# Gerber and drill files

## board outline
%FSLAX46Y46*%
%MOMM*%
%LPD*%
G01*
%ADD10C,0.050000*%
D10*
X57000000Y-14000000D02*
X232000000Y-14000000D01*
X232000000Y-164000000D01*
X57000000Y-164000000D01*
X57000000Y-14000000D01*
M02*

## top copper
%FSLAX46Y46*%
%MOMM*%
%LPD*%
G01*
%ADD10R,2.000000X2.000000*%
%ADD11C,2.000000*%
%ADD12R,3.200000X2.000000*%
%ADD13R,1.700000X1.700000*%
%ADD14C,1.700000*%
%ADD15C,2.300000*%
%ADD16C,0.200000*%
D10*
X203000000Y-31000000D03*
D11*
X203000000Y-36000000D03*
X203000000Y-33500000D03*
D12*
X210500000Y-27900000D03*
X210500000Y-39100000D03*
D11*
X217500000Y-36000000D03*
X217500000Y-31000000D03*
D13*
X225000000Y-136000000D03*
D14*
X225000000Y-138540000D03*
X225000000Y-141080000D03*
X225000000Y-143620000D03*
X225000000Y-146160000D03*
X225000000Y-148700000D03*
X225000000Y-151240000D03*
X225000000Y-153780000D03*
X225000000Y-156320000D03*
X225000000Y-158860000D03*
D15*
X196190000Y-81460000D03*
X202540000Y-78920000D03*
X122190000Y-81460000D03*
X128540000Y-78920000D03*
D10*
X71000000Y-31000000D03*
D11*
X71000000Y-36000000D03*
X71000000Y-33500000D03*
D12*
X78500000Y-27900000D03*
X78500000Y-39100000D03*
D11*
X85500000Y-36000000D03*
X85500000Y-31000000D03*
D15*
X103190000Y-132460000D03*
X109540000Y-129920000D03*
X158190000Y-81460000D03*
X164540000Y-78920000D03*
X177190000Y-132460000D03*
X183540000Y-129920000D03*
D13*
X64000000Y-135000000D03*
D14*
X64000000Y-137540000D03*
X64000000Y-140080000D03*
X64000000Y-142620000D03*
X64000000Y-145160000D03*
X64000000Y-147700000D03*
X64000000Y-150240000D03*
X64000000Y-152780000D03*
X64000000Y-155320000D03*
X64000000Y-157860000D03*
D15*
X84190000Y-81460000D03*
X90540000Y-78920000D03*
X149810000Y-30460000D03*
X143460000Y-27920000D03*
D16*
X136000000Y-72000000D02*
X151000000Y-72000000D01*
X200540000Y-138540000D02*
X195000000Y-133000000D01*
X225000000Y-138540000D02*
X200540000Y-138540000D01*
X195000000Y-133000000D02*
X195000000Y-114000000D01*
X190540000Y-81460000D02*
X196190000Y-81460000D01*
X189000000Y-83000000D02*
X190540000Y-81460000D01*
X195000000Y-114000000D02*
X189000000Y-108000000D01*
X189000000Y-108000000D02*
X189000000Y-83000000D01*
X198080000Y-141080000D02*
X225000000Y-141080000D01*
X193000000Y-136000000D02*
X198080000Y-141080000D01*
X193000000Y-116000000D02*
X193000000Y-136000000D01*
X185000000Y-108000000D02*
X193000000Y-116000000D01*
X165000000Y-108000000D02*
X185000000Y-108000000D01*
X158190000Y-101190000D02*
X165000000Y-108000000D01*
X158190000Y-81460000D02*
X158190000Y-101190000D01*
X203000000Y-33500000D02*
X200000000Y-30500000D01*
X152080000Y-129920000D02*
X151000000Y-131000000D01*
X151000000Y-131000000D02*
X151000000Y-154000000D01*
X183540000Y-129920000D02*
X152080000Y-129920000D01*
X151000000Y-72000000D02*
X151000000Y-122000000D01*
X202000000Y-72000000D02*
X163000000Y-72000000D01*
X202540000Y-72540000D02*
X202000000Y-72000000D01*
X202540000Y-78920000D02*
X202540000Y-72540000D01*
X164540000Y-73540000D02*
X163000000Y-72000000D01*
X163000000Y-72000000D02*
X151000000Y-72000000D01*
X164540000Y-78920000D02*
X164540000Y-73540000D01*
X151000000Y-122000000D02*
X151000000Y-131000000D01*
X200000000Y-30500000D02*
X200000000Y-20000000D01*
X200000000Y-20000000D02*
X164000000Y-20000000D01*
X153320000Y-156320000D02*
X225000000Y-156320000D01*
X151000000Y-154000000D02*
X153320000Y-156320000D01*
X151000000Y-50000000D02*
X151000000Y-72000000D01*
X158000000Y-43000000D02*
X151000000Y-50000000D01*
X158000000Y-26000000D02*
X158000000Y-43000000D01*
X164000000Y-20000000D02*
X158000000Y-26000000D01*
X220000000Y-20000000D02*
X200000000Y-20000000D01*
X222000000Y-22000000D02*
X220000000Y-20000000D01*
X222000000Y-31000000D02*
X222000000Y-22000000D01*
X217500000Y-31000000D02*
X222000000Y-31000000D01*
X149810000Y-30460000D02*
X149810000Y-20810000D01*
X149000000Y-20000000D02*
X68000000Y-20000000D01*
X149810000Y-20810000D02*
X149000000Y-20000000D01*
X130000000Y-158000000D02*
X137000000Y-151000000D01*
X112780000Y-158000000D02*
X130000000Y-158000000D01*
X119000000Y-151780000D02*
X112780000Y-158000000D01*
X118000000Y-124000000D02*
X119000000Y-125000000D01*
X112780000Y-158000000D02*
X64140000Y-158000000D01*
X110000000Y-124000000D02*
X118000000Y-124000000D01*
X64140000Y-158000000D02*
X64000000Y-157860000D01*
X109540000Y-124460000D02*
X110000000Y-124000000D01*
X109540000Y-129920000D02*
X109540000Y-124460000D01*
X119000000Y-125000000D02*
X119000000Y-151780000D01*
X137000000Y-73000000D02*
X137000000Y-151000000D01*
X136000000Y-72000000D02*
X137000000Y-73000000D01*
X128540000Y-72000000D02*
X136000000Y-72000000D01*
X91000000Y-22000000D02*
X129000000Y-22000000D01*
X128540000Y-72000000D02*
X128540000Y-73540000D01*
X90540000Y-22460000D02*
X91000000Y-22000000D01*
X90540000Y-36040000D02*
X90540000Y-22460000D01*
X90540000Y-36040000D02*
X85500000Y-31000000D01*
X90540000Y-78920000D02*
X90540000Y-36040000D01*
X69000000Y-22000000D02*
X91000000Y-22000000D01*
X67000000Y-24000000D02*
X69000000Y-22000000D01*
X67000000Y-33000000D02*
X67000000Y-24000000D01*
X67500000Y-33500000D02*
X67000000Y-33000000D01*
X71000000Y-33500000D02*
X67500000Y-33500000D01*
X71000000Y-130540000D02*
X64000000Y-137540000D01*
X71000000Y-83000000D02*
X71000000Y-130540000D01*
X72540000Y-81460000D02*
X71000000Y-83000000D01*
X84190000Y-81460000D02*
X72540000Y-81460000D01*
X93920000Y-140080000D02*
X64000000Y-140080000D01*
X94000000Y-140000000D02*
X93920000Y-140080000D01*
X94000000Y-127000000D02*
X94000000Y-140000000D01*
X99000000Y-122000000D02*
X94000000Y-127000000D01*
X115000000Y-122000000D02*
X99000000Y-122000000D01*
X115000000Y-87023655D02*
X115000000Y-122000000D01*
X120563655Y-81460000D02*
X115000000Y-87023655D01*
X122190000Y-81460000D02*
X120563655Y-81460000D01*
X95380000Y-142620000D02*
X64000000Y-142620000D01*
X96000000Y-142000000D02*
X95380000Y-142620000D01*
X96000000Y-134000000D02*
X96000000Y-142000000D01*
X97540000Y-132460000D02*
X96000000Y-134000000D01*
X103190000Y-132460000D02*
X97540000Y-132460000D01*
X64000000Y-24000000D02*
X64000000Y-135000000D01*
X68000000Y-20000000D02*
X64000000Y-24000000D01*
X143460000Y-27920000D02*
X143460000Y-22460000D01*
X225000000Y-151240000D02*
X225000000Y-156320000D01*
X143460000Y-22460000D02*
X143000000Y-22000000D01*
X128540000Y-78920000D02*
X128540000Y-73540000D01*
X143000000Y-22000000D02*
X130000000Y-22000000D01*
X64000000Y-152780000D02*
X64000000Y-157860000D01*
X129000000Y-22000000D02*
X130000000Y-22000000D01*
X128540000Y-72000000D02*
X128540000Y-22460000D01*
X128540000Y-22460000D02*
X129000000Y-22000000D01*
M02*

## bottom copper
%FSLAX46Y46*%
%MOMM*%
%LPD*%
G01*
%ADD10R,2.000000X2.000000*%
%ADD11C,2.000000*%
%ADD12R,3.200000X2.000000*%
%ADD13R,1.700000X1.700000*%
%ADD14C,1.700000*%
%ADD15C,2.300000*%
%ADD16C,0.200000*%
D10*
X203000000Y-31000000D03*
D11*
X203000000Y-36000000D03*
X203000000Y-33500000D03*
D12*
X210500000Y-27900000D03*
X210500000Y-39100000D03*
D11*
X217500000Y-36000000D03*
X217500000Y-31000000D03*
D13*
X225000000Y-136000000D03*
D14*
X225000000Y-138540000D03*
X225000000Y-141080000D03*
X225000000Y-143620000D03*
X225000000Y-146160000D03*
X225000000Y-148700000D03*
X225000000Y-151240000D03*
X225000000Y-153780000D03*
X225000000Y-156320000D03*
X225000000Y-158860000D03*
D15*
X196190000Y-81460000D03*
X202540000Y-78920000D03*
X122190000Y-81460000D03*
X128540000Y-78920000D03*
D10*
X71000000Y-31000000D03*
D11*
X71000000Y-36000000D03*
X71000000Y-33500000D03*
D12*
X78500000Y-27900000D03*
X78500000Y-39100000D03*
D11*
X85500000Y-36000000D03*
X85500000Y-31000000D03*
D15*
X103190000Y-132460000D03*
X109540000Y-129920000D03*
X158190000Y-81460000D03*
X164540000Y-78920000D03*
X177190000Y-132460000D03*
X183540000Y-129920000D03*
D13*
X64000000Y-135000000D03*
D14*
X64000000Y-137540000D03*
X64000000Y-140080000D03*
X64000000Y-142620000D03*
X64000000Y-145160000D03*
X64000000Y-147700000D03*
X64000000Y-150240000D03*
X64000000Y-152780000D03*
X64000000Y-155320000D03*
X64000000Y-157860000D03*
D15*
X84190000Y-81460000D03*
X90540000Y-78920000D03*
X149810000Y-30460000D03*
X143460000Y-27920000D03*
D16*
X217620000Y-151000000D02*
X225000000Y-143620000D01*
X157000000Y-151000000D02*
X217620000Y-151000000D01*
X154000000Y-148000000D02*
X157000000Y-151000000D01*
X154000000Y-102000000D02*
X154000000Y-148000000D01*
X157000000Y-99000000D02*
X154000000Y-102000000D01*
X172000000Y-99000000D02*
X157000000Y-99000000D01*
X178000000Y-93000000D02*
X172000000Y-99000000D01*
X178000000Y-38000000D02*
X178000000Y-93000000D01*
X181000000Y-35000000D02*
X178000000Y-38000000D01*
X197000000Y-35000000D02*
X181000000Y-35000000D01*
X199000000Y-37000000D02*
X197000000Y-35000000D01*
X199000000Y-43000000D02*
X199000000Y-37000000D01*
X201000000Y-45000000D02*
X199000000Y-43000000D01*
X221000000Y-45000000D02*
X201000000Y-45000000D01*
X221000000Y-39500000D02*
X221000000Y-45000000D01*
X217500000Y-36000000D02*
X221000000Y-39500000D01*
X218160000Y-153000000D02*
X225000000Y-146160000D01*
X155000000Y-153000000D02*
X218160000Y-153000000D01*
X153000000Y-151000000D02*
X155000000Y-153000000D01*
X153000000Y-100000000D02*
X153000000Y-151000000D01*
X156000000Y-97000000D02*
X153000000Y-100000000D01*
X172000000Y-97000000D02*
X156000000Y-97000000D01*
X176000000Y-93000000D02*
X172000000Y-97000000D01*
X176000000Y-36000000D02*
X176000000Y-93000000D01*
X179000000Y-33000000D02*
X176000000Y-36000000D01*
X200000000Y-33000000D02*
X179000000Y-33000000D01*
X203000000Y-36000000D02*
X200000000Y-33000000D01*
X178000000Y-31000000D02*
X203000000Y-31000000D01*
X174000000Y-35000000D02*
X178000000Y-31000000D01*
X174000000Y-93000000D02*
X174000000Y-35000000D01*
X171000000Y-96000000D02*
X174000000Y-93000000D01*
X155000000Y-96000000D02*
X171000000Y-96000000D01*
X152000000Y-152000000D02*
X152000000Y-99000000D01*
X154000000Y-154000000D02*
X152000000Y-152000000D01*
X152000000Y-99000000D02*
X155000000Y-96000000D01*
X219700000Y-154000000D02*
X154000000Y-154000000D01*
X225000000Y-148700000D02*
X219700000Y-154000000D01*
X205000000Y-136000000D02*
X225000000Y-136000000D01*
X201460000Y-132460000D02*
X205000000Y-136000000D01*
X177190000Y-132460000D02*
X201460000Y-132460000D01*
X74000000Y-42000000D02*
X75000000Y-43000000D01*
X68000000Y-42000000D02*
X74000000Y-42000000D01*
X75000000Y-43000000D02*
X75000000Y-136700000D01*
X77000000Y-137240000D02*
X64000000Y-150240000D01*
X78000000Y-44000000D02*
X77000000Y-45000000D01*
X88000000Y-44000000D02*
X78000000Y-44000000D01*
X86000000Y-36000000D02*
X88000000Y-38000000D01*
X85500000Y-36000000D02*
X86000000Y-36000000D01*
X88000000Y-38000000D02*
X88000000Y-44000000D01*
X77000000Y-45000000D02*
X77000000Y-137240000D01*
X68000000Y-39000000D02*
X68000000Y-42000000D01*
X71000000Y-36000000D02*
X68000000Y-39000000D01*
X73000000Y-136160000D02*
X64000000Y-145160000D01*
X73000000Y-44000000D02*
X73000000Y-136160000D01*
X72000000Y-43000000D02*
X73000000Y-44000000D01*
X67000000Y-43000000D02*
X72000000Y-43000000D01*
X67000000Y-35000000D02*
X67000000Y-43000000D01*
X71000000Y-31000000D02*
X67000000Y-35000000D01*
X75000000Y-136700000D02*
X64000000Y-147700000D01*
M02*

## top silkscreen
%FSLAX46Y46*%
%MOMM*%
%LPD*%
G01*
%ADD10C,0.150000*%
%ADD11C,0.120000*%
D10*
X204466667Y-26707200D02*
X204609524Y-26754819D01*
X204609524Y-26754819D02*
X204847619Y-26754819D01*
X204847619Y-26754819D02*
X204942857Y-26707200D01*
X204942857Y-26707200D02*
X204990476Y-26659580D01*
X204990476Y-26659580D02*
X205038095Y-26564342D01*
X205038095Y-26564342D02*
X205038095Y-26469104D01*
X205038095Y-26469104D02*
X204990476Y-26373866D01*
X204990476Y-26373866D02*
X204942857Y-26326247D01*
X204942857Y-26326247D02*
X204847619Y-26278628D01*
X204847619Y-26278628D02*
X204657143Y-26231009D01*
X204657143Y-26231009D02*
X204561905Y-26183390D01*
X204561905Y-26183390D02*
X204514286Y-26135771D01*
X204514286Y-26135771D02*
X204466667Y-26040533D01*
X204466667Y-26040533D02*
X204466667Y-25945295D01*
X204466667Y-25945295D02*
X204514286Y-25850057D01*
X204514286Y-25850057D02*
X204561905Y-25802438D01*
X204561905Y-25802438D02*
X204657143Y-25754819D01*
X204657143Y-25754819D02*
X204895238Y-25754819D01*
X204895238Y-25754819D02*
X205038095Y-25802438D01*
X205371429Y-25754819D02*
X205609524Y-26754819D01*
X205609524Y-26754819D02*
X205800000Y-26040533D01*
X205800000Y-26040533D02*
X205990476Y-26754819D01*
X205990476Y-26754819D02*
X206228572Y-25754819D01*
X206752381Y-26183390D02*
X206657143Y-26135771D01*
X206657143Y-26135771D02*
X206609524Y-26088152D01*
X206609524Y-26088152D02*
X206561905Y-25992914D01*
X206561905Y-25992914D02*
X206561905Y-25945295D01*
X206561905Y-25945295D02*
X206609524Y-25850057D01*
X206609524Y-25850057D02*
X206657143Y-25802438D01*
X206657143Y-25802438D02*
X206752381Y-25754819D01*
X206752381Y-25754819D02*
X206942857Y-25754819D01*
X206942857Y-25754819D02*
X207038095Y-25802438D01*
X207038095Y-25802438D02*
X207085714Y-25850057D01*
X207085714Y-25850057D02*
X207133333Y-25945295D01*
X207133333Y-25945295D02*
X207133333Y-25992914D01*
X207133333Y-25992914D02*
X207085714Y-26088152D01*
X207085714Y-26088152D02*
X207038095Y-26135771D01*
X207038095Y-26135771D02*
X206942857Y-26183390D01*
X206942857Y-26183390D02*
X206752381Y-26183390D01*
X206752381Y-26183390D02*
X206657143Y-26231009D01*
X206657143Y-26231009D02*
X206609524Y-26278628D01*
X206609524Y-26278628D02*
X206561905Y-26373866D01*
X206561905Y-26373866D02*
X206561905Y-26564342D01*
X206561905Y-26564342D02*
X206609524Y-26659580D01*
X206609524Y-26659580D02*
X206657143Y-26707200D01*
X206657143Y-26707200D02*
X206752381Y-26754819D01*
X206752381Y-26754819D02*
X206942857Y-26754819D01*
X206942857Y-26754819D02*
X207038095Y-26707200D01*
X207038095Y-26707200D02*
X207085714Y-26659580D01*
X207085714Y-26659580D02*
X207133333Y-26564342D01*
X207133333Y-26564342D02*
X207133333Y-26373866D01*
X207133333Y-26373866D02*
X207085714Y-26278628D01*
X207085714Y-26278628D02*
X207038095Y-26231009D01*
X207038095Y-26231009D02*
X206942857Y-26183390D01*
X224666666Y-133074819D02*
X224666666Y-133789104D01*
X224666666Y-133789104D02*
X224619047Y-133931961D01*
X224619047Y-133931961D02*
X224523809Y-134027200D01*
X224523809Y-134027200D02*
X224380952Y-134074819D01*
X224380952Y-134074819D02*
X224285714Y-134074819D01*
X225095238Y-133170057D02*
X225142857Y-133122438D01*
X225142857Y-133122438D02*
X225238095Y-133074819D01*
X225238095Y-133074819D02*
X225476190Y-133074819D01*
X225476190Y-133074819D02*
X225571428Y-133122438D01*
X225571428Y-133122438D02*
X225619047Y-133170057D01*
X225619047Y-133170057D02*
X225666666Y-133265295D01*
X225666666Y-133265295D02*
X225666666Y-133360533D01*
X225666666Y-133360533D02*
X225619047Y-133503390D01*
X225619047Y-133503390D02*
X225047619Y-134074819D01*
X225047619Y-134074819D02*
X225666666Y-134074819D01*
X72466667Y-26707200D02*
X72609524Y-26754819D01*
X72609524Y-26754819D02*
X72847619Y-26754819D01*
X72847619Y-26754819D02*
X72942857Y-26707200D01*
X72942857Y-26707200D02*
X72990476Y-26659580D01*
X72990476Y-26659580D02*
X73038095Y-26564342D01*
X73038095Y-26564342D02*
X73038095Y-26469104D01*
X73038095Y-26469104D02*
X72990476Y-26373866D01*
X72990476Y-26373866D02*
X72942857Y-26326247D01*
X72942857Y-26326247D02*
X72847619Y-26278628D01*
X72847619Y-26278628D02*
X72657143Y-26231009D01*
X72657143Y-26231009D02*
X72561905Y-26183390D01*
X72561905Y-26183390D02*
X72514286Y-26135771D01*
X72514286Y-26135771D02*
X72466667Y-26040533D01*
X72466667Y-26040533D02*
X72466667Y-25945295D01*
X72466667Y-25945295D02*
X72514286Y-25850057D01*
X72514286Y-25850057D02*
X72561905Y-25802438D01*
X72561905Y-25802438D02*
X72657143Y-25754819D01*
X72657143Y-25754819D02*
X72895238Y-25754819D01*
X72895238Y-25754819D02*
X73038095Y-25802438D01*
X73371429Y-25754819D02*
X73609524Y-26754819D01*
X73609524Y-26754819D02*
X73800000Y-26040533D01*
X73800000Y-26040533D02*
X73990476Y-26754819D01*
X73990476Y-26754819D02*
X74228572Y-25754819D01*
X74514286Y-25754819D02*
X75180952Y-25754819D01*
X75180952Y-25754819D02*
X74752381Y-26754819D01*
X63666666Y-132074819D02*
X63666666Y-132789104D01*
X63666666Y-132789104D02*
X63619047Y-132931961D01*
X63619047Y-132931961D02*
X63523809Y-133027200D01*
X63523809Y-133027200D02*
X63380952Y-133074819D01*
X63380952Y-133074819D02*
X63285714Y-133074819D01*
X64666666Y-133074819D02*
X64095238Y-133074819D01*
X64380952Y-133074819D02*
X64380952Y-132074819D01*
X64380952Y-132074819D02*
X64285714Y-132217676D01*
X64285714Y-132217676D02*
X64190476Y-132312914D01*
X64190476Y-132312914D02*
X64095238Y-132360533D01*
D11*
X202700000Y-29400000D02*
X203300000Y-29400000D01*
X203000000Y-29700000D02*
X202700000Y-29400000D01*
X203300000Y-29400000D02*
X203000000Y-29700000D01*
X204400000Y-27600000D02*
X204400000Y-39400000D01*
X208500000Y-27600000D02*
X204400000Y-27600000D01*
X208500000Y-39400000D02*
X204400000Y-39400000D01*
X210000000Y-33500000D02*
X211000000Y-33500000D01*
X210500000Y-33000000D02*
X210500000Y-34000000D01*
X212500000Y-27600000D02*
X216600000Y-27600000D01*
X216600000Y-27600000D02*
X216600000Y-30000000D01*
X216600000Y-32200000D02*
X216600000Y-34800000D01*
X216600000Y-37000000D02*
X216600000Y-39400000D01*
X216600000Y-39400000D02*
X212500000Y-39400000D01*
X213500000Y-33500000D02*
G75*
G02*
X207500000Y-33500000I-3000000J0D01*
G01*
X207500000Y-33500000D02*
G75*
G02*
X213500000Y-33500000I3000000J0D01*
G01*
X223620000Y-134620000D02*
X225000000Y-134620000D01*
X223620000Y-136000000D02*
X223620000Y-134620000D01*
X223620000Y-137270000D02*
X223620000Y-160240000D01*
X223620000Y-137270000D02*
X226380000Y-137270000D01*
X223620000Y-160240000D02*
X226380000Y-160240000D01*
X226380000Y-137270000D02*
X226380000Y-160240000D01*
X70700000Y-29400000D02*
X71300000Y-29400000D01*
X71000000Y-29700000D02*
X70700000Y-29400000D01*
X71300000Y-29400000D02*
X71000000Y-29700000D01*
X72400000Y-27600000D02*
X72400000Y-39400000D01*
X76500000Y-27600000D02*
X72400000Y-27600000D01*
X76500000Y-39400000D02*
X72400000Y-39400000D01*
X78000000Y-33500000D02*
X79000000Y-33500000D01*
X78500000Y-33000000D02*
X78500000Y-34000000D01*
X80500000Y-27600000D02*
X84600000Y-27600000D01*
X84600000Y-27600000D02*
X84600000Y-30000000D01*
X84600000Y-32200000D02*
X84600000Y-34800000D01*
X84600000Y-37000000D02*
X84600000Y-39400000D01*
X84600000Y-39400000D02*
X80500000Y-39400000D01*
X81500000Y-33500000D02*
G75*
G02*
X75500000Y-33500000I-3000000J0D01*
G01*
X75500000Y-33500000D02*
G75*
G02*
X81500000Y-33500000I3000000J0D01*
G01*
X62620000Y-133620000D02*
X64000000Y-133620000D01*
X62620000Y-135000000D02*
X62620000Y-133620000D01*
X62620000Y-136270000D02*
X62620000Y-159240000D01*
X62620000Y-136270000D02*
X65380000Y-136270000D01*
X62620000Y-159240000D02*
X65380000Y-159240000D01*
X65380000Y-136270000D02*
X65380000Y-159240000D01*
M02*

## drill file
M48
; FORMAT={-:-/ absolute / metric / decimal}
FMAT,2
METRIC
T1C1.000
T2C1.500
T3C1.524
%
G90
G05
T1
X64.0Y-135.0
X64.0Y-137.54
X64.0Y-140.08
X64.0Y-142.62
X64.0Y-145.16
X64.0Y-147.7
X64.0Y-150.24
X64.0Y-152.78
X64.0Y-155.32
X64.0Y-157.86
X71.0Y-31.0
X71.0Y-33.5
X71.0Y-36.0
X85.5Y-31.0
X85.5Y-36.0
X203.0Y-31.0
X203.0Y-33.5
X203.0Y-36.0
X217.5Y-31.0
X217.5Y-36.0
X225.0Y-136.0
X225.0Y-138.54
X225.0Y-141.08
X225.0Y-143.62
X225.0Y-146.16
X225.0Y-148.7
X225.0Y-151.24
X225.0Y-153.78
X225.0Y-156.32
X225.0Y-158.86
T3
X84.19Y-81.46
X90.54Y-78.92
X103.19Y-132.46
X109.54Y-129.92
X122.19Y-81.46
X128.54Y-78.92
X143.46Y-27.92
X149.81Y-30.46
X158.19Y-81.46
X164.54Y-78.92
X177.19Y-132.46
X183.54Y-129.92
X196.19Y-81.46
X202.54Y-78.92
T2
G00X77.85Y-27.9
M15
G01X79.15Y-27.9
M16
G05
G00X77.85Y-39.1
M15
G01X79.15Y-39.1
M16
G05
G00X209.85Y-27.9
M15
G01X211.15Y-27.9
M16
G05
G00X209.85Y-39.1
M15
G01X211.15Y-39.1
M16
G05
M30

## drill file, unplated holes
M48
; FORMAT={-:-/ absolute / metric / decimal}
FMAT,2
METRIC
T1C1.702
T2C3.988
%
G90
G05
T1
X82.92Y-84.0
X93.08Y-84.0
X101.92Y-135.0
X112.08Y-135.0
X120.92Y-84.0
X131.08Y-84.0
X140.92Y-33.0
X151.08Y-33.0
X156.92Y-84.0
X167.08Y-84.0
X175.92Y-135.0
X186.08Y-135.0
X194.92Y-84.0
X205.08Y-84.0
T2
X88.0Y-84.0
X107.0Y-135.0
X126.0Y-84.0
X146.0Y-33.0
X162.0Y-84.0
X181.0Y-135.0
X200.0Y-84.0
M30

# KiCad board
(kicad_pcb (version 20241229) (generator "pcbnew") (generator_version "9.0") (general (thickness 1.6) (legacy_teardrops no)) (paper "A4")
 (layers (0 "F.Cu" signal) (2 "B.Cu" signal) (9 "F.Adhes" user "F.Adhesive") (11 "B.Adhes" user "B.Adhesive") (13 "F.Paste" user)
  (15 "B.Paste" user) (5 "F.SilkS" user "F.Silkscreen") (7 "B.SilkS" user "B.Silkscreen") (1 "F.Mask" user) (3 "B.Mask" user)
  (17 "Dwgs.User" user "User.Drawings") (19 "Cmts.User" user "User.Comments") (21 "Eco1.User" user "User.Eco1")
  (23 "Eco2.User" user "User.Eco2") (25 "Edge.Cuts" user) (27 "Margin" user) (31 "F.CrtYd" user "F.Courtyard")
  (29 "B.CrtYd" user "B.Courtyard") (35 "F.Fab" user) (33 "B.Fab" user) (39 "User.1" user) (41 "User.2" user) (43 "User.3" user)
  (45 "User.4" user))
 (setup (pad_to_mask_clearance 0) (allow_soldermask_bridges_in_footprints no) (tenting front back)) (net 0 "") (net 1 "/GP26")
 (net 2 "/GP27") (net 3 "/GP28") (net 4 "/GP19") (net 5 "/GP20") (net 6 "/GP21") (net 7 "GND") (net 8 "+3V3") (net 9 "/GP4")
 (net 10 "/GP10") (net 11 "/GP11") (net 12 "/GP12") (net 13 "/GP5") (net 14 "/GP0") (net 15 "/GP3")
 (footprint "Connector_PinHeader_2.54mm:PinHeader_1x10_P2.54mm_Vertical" (layer "F.Cu") (at 225 136)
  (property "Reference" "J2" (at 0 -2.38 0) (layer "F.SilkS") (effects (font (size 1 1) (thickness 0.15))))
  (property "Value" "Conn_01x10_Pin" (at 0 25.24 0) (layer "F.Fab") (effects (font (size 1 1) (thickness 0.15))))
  (fp_line (start -1.38 -1.38) (end 0 -1.38) (stroke (width 0.12) (type solid)) (layer "F.SilkS"))
  (fp_line (start -1.38 0) (end -1.38 -1.38) (stroke (width 0.12) (type solid)) (layer "F.SilkS"))
  (fp_line (start -1.38 1.27) (end -1.38 24.24) (stroke (width 0.12) (type solid)) (layer "F.SilkS"))
  (fp_line (start -1.38 1.27) (end 1.38 1.27) (stroke (width 0.12) (type solid)) (layer "F.SilkS"))
  (fp_line (start -1.38 24.24) (end 1.38 24.24) (stroke (width 0.12) (type solid)) (layer "F.SilkS"))
  (fp_line (start 1.38 1.27) (end 1.38 24.24) (stroke (width 0.12) (type solid)) (layer "F.SilkS"))
  (pad "1" thru_hole rect (at 0 0) (size 1.7 1.7) (drill 1) (layers "*.Cu" "*.Mask") (remove_unused_layers no) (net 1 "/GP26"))
  (pad "2" thru_hole circle (at 0 2.54) (size 1.7 1.7) (drill 1) (layers "*.Cu" "*.Mask") (remove_unused_layers no) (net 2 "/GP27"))
  (pad "3" thru_hole circle (at 0 5.08) (size 1.7 1.7) (drill 1) (layers "*.Cu" "*.Mask") (remove_unused_layers no) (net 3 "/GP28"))
  (pad "4" thru_hole circle (at 0 7.62) (size 1.7 1.7) (drill 1) (layers "*.Cu" "*.Mask") (remove_unused_layers no) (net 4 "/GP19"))
  (pad "5" thru_hole circle (at 0 10.16) (size 1.7 1.7) (drill 1) (layers "*.Cu" "*.Mask") (remove_unused_layers no) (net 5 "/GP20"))
  (pad "6" thru_hole circle (at 0 12.7) (size 1.7 1.7) (drill 1) (layers "*.Cu" "*.Mask") (remove_unused_layers no) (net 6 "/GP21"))
  (pad "7" thru_hole circle (at 0 15.24) (size 1.7 1.7) (drill 1) (layers "*.Cu" "*.Mask") (remove_unused_layers no) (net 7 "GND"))
  (pad "8" thru_hole circle (at 0 17.78) (size 1.7 1.7) (drill 1) (layers "*.Cu" "*.Mask") (remove_unused_layers no) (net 7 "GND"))
  (pad "9" thru_hole circle (at 0 20.32) (size 1.7 1.7) (drill 1) (layers "*.Cu" "*.Mask") (remove_unused_layers no) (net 7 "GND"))
  (pad "10" thru_hole circle (at 0 22.86) (size 1.7 1.7) (drill 1) (layers "*.Cu" "*.Mask") (remove_unused_layers no) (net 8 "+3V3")))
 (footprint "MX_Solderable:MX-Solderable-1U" (layer "F.Cu") (at 200 84)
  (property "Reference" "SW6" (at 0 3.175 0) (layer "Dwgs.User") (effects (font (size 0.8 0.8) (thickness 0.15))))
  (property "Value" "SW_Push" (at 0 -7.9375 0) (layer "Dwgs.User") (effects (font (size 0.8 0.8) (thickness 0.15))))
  (pad "" np_thru_hole circle (at -5.08 0 48.099) (size 1.7018 1.7018) (drill 1.7018) (layers "*.Cu" "*.Mask"))
  (pad "" np_thru_hole circle (at 0 0) (size 3.9878 3.9878) (drill 3.9878) (layers "*.Cu" "*.Mask"))
  (pad "" np_thru_hole circle (at 5.08 0 48.099) (size 1.7018 1.7018) (drill 1.7018) (layers "*.Cu" "*.Mask"))
  (pad "1" thru_hole circle (at -3.81 -2.54) (size 2.3 2.3) (drill 1.524) (layers "*.Cu" "B.Mask") (remove_unused_layers no) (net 2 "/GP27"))
  (pad "2" thru_hole circle (at 2.54 -5.08) (size 2.3 2.3) (drill 1.524) (layers "*.Cu" "B.Mask") (remove_unused_layers no) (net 7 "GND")))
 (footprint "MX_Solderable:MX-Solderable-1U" (layer "F.Cu") (at 126 84)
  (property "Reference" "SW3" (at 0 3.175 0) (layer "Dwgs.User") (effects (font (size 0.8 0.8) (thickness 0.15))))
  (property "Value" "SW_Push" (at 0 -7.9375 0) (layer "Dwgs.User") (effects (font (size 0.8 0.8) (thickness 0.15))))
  (pad "" np_thru_hole circle (at -5.08 0 48.099) (size 1.7018 1.7018) (drill 1.7018) (layers "*.Cu" "*.Mask"))
  (pad "" np_thru_hole circle (at 0 0) (size 3.9878 3.9878) (drill 3.9878) (layers "*.Cu" "*.Mask"))
  (pad "" np_thru_hole circle (at 5.08 0 48.099) (size 1.7018 1.7018) (drill 1.7018) (layers "*.Cu" "*.Mask"))
  (pad "1" thru_hole circle (at -3.81 -2.54) (size 2.3 2.3) (drill 1.524) (layers "*.Cu" "B.Mask") (remove_unused_layers no) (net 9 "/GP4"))
  (pad "2" thru_hole circle (at 2.54 -5.08) (size 2.3 2.3) (drill 1.524) (layers "*.Cu" "B.Mask") (remove_unused_layers no) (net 7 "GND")))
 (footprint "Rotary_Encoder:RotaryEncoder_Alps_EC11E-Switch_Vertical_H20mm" (layer "F.Cu") (at 71 31)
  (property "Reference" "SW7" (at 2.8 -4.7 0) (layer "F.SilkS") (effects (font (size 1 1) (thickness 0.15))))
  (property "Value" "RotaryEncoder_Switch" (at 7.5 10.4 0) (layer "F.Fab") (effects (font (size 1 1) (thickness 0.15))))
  (fp_line (start -0.3 -1.6) (end 0.3 -1.6) (stroke (width 0.12) (type solid)) (layer "F.SilkS"))
  (fp_line (start 0 -1.3) (end -0.3 -1.6) (stroke (width 0.12) (type solid)) (layer "F.SilkS"))
  (fp_line (start 0.3 -1.6) (end 0 -1.3) (stroke (width 0.12) (type solid)) (layer "F.SilkS"))
  (fp_line (start 1.4 -3.4) (end 1.4 8.4) (stroke (width 0.12) (type solid)) (layer "F.SilkS"))
  (fp_line (start 5.5 -3.4) (end 1.4 -3.4) (stroke (width 0.12) (type solid)) (layer "F.SilkS"))
  (fp_line (start 5.5 8.4) (end 1.4 8.4) (stroke (width 0.12) (type solid)) (layer "F.SilkS"))
  (fp_line (start 7 2.5) (end 8 2.5) (stroke (width 0.12) (type solid)) (layer "F.SilkS"))
  (fp_line (start 7.5 2) (end 7.5 3) (stroke (width 0.12) (type solid)) (layer "F.SilkS"))
  (fp_line (start 9.5 -3.4) (end 13.6 -3.4) (stroke (width 0.12) (type solid)) (layer "F.SilkS"))
  (fp_line (start 13.6 -3.4) (end 13.6 -1) (stroke (width 0.12) (type solid)) (layer "F.SilkS"))
  (fp_line (start 13.6 1.2) (end 13.6 3.8) (stroke (width 0.12) (type solid)) (layer "F.SilkS"))
  (fp_line (start 13.6 6) (end 13.6 8.4) (stroke (width 0.12) (type solid)) (layer "F.SilkS"))
  (fp_line (start 13.6 8.4) (end 9.5 8.4) (stroke (width 0.12) (type solid)) (layer "F.SilkS"))
  (fp_circle (center 7.5 2.5) (end 10.5 2.5) (stroke (width 0.12) (type solid)) (fill no) (layer "F.SilkS"))
  (pad "A" thru_hole rect (at 0 0) (size 2 2) (drill 1) (layers "*.Cu" "*.Mask") (remove_unused_layers no) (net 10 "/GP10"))
  (pad "B" thru_hole circle (at 0 5) (size 2 2) (drill 1) (layers "*.Cu" "*.Mask") (remove_unused_layers no) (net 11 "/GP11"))
  (pad "C" thru_hole circle (at 0 2.5) (size 2 2) (drill 1) (layers "*.Cu" "*.Mask") (remove_unused_layers no) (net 7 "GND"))
  (pad "MP" thru_hole rect (at 7.5 -3.1) (size 3.2 2) (drill oval 2.8 1.5) (layers "*.Cu" "*.Mask") (remove_unused_layers no))
  (pad "MP" thru_hole rect (at 7.5 8.1) (size 3.2 2) (drill oval 2.8 1.5) (layers "*.Cu" "*.Mask") (remove_unused_layers no))
  (pad "S1" thru_hole circle (at 14.5 5) (size 2 2) (drill 1) (layers "*.Cu" "*.Mask") (remove_unused_layers no) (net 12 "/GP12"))
  (pad "S2" thru_hole circle (at 14.5 0) (size 2 2) (drill 1) (layers "*.Cu" "*.Mask") (remove_unused_layers no) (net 7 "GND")))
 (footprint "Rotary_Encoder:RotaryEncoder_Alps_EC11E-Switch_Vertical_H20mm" (layer "F.Cu") (at 203 31)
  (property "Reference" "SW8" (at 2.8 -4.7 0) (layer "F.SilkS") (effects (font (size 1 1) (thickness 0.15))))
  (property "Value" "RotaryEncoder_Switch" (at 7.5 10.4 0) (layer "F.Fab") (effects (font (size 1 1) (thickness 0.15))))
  (fp_line (start -0.3 -1.6) (end 0.3 -1.6) (stroke (width 0.12) (type solid)) (layer "F.SilkS"))
  (fp_line (start 0 -1.3) (end -0.3 -1.6) (stroke (width 0.12) (type solid)) (layer "F.SilkS"))
  (fp_line (start 0.3 -1.6) (end 0 -1.3) (stroke (width 0.12) (type solid)) (layer "F.SilkS"))
  (fp_line (start 1.4 -3.4) (end 1.4 8.4) (stroke (width 0.12) (type solid)) (layer "F.SilkS"))
  (fp_line (start 5.5 -3.4) (end 1.4 -3.4) (stroke (width 0.12) (type solid)) (layer "F.SilkS"))
  (fp_line (start 5.5 8.4) (end 1.4 8.4) (stroke (width 0.12) (type solid)) (layer "F.SilkS"))
  (fp_line (start 7 2.5) (end 8 2.5) (stroke (width 0.12) (type solid)) (layer "F.SilkS"))
  (fp_line (start 7.5 2) (end 7.5 3) (stroke (width 0.12) (type solid)) (layer "F.SilkS"))
  (fp_line (start 9.5 -3.4) (end 13.6 -3.4) (stroke (width 0.12) (type solid)) (layer "F.SilkS"))
  (fp_line (start 13.6 -3.4) (end 13.6 -1) (stroke (width 0.12) (type solid)) (layer "F.SilkS"))
  (fp_line (start 13.6 1.2) (end 13.6 3.8) (stroke (width 0.12) (type solid)) (layer "F.SilkS"))
  (fp_line (start 13.6 6) (end 13.6 8.4) (stroke (width 0.12) (type solid)) (layer "F.SilkS"))
  (fp_line (start 13.6 8.4) (end 9.5 8.4) (stroke (width 0.12) (type solid)) (layer "F.SilkS"))
  (fp_circle (center 7.5 2.5) (end 10.5 2.5) (stroke (width 0.12) (type solid)) (fill no) (layer "F.SilkS"))
  (pad "A" thru_hole rect (at 0 0) (size 2 2) (drill 1) (layers "*.Cu" "*.Mask") (remove_unused_layers no) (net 6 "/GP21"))
  (pad "B" thru_hole circle (at 0 5) (size 2 2) (drill 1) (layers "*.Cu" "*.Mask") (remove_unused_layers no) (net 5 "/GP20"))
  (pad "C" thru_hole circle (at 0 2.5) (size 2 2) (drill 1) (layers "*.Cu" "*.Mask") (remove_unused_layers no) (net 7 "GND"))
  (pad "MP" thru_hole rect (at 7.5 -3.1) (size 3.2 2) (drill oval 2.8 1.5) (layers "*.Cu" "*.Mask") (remove_unused_layers no))
  (pad "MP" thru_hole rect (at 7.5 8.1) (size 3.2 2) (drill oval 2.8 1.5) (layers "*.Cu" "*.Mask") (remove_unused_layers no))
  (pad "S1" thru_hole circle (at 14.5 5) (size 2 2) (drill 1) (layers "*.Cu" "*.Mask") (remove_unused_layers no) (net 4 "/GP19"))
  (pad "S2" thru_hole circle (at 14.5 0) (size 2 2) (drill 1) (layers "*.Cu" "*.Mask") (remove_unused_layers no) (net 7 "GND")))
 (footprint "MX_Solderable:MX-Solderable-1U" (layer "F.Cu") (at 107 135)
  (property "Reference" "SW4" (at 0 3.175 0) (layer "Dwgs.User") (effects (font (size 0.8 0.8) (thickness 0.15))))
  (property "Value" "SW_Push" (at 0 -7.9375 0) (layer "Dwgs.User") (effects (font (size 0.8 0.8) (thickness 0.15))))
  (pad "" np_thru_hole circle (at -5.08 0 48.099) (size 1.7018 1.7018) (drill 1.7018) (layers "*.Cu" "*.Mask"))
  (pad "" np_thru_hole circle (at 0 0) (size 3.9878 3.9878) (drill 3.9878) (layers "*.Cu" "*.Mask"))
  (pad "" np_thru_hole circle (at 5.08 0 48.099) (size 1.7018 1.7018) (drill 1.7018) (layers "*.Cu" "*.Mask"))
  (pad "1" thru_hole circle (at -3.81 -2.54) (size 2.3 2.3) (drill 1.524) (layers "*.Cu" "B.Mask") (remove_unused_layers no) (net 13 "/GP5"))
  (pad "2" thru_hole circle (at 2.54 -5.08) (size 2.3 2.3) (drill 1.524) (layers "*.Cu" "B.Mask") (remove_unused_layers no) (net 7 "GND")))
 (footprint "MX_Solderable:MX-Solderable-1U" (layer "F.Cu") (at 162 84)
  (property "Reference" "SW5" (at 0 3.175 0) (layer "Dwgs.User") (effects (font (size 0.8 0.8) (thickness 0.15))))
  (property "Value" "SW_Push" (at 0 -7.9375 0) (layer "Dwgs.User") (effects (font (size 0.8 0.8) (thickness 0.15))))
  (pad "" np_thru_hole circle (at -5.08 0 48.099) (size 1.7018 1.7018) (drill 1.7018) (layers "*.Cu" "*.Mask"))
  (pad "" np_thru_hole circle (at 0 0) (size 3.9878 3.9878) (drill 3.9878) (layers "*.Cu" "*.Mask"))
  (pad "" np_thru_hole circle (at 5.08 0 48.099) (size 1.7018 1.7018) (drill 1.7018) (layers "*.Cu" "*.Mask"))
  (pad "1" thru_hole circle (at -3.81 -2.54) (size 2.3 2.3) (drill 1.524) (layers "*.Cu" "B.Mask") (remove_unused_layers no) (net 3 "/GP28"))
  (pad "2" thru_hole circle (at 2.54 -5.08) (size 2.3 2.3) (drill 1.524) (layers "*.Cu" "B.Mask") (remove_unused_layers no) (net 7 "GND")))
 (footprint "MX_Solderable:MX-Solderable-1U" (layer "F.Cu") (at 181 135)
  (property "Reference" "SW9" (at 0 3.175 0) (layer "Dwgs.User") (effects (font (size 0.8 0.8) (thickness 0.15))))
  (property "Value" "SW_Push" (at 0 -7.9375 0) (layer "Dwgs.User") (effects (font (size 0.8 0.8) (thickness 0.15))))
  (pad "" np_thru_hole circle (at -5.08 0 48.099) (size 1.7018 1.7018) (drill 1.7018) (layers "*.Cu" "*.Mask"))
  (pad "" np_thru_hole circle (at 0 0) (size 3.9878 3.9878) (drill 3.9878) (layers "*.Cu" "*.Mask"))
  (pad "" np_thru_hole circle (at 5.08 0 48.099) (size 1.7018 1.7018) (drill 1.7018) (layers "*.Cu" "*.Mask"))
  (pad "1" thru_hole circle (at -3.81 -2.54) (size 2.3 2.3) (drill 1.524) (layers "*.Cu" "B.Mask") (remove_unused_layers no) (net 1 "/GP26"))
  (pad "2" thru_hole circle (at 2.54 -5.08) (size 2.3 2.3) (drill 1.524) (layers "*.Cu" "B.Mask") (remove_unused_layers no) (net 7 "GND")))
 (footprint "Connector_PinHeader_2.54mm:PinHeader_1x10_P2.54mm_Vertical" (layer "F.Cu") (at 64 135)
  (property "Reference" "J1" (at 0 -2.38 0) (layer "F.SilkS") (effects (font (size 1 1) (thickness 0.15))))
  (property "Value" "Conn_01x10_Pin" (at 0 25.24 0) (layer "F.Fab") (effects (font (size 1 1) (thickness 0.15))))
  (fp_line (start -1.38 -1.38) (end 0 -1.38) (stroke (width 0.12) (type solid)) (layer "F.SilkS"))
  (fp_line (start -1.38 0) (end -1.38 -1.38) (stroke (width 0.12) (type solid)) (layer "F.SilkS"))
  (fp_line (start -1.38 1.27) (end -1.38 24.24) (stroke (width 0.12) (type solid)) (layer "F.SilkS"))
  (fp_line (start -1.38 1.27) (end 1.38 1.27) (stroke (width 0.12) (type solid)) (layer "F.SilkS"))
  (fp_line (start -1.38 24.24) (end 1.38 24.24) (stroke (width 0.12) (type solid)) (layer "F.SilkS"))
  (fp_line (start 1.38 1.27) (end 1.38 24.24) (stroke (width 0.12) (type solid)) (layer "F.SilkS"))
  (pad "1" thru_hole rect (at 0 0) (size 1.7 1.7) (drill 1) (layers "*.Cu" "*.Mask") (remove_unused_layers no) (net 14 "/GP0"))
  (pad "2" thru_hole circle (at 0 2.54) (size 1.7 1.7) (drill 1) (layers "*.Cu" "*.Mask") (remove_unused_layers no) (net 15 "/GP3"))
  (pad "3" thru_hole circle (at 0 5.08) (size 1.7 1.7) (drill 1) (layers "*.Cu" "*.Mask") (remove_unused_layers no) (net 9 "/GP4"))
  (pad "4" thru_hole circle (at 0 7.62) (size 1.7 1.7) (drill 1) (layers "*.Cu" "*.Mask") (remove_unused_layers no) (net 13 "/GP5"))
  (pad "5" thru_hole circle (at 0 10.16) (size 1.7 1.7) (drill 1) (layers "*.Cu" "*.Mask") (remove_unused_layers no) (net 10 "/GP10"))
  (pad "6" thru_hole circle (at 0 12.7) (size 1.7 1.7) (drill 1) (layers "*.Cu" "*.Mask") (remove_unused_layers no) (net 11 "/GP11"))
  (pad "7" thru_hole circle (at 0 15.24) (size 1.7 1.7) (drill 1) (layers "*.Cu" "*.Mask") (remove_unused_layers no) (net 12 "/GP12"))
  (pad "8" thru_hole circle (at 0 17.78) (size 1.7 1.7) (drill 1) (layers "*.Cu" "*.Mask") (remove_unused_layers no) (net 7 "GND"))
  (pad "9" thru_hole circle (at 0 20.32) (size 1.7 1.7) (drill 1) (layers "*.Cu" "*.Mask") (remove_unused_layers no) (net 7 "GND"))
  (pad "10" thru_hole circle (at 0 22.86) (size 1.7 1.7) (drill 1) (layers "*.Cu" "*.Mask") (remove_unused_layers no) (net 7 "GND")))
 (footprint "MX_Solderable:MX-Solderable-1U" (layer "F.Cu") (at 88 84)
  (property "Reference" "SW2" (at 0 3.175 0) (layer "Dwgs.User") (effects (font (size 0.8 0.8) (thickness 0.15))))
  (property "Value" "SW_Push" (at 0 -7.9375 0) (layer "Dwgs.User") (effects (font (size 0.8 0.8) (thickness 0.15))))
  (pad "" np_thru_hole circle (at -5.08 0 48.099) (size 1.7018 1.7018) (drill 1.7018) (layers "*.Cu" "*.Mask"))
  (pad "" np_thru_hole circle (at 0 0) (size 3.9878 3.9878) (drill 3.9878) (layers "*.Cu" "*.Mask"))
  (pad "" np_thru_hole circle (at 5.08 0 48.099) (size 1.7018 1.7018) (drill 1.7018) (layers "*.Cu" "*.Mask"))
  (pad "1" thru_hole circle (at -3.81 -2.54) (size 2.3 2.3) (drill 1.524) (layers "*.Cu" "B.Mask") (remove_unused_layers no) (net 15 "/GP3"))
  (pad "2" thru_hole circle (at 2.54 -5.08) (size 2.3 2.3) (drill 1.524) (layers "*.Cu" "B.Mask") (remove_unused_layers no) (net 7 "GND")))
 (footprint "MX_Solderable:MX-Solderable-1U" (layer "B.Cu") (at 146 33 180)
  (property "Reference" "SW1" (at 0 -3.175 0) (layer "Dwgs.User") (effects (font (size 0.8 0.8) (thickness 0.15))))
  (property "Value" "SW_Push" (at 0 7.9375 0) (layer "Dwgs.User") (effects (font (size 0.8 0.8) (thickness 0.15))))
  (pad "" np_thru_hole circle (at -5.08 0 131.901) (size 1.7018 1.7018) (drill 1.7018) (layers "*.Cu" "*.Mask"))
  (pad "" np_thru_hole circle (at 0 0 180) (size 3.9878 3.9878) (drill 3.9878) (layers "*.Cu" "*.Mask"))
  (pad "" np_thru_hole circle (at 5.08 0 131.901) (size 1.7018 1.7018) (drill 1.7018) (layers "*.Cu" "*.Mask"))
  (pad "1" thru_hole circle (at -3.81 2.54 180) (size 2.3 2.3) (drill 1.524) (layers "*.Cu" "F.Mask") (remove_unused_layers no)
   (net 14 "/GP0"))
  (pad "2" thru_hole circle (at 2.54 5.08 180) (size 2.3 2.3) (drill 1.524) (layers "*.Cu" "F.Mask") (remove_unused_layers no) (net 7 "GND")))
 (gr_rect (start 57 14) (end 232 164) (stroke (width 0.05) (type solid)) (fill no) (layer "Edge.Cuts"))
 (segment (start 77 45) (end 77 137.24) (width 0.2) (layer "B.Cu") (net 12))
 (segment (start 77 137.24) (end 64 150.24) (width 0.2) (layer "B.Cu") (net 12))
 (segment (start 88 44) (end 78 44) (width 0.2) (layer "B.Cu") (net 12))
 (segment (start 85.5 36) (end 86 36) (width 0.2) (layer "B.Cu") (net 12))
 (segment (start 86 36) (end 88 38) (width 0.2) (layer "B.Cu") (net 12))
 (segment (start 78 44) (end 77 45) (width 0.2) (layer "B.Cu") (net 12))
 (segment (start 88 38) (end 88 44) (width 0.2) (layer "B.Cu") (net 12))
 (segment (start 158 26) (end 158 43) (width 0.2) (layer "F.Cu") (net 7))
 (segment (start 202.54 78.92) (end 202.54 72.54) (width 0.2) (layer "F.Cu") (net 7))
 (segment (start 137 73) (end 137 151) (width 0.2) (layer "F.Cu") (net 7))
 (segment (start 143.46 27.92) (end 143.46 22.46) (width 0.2) (layer "F.Cu") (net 7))
 (segment (start 158 43) (end 151 50) (width 0.2) (layer "F.Cu") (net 7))
 (segment (start 202 72) (end 163 72) (width 0.2) (layer "F.Cu") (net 7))
 (segment (start 153.32 156.32) (end 225 156.32) (width 0.2) (layer "F.Cu") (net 7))
 (segment (start 151 154) (end 153.32 156.32) (width 0.2) (layer "F.Cu") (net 7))
 (segment (start 136 72) (end 151 72) (width 0.2) (layer "F.Cu") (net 7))
 (segment (start 64.14 158) (end 64 157.86) (width 0.2) (layer "F.Cu") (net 7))
 (segment (start 71 33.5) (end 67.5 33.5) (width 0.2) (layer "F.Cu") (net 7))
 (segment (start 128.54 72) (end 128.54 22.46) (width 0.2) (layer "F.Cu") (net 7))
 (segment (start 217.5 31) (end 222 31) (width 0.2) (layer "F.Cu") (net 7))
 (segment (start 225 151.24) (end 225 156.32) (width 0.2) (layer "F.Cu") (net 7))
 (segment (start 67.5 33.5) (end 67 33) (width 0.2) (layer "F.Cu") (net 7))
 (segment (start 90.54 22.46) (end 91 22) (width 0.2) (layer "F.Cu") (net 7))
 (segment (start 109.54 124.46) (end 110 124) (width 0.2) (layer "F.Cu") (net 7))
 (segment (start 67 33) (end 67 24) (width 0.2) (layer "F.Cu") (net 7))
 (segment (start 163 72) (end 151 72) (width 0.2) (layer "F.Cu") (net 7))
 (segment (start 164.54 73.54) (end 163 72) (width 0.2) (layer "F.Cu") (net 7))
 (segment (start 130 158) (end 137 151) (width 0.2) (layer "F.Cu") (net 7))
 (segment (start 164 20) (end 158 26) (width 0.2) (layer "F.Cu") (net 7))
 (segment (start 69 22) (end 91 22) (width 0.2) (layer "F.Cu") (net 7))
 (segment (start 112.78 158) (end 130 158) (width 0.2) (layer "F.Cu") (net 7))
 (segment (start 136 72) (end 137 73) (width 0.2) (layer "F.Cu") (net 7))
 (segment (start 151 72) (end 151 122) (width 0.2) (layer "F.Cu") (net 7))
 (segment (start 90.54 36.04) (end 90.54 22.46) (width 0.2) (layer "F.Cu") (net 7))
 (segment (start 200 20) (end 164 20) (width 0.2) (layer "F.Cu") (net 7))
 (segment (start 67 24) (end 69 22) (width 0.2) (layer "F.Cu") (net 7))
 (segment (start 128.54 72) (end 136 72) (width 0.2) (layer "F.Cu") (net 7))
 (segment (start 151 122) (end 151 131) (width 0.2) (layer "F.Cu") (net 7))
 (segment (start 90.54 36.04) (end 85.5 31) (width 0.2) (layer "F.Cu") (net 7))
 (segment (start 203 33.5) (end 200 30.5) (width 0.2) (layer "F.Cu") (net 7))
 (segment (start 128.54 22.46) (end 129 22) (width 0.2) (layer "F.Cu") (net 7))
 (segment (start 112.78 158) (end 64.14 158) (width 0.2) (layer "F.Cu") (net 7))
 (segment (start 143.46 22.46) (end 143 22) (width 0.2) (layer "F.Cu") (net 7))
 (segment (start 109.54 129.92) (end 109.54 124.46) (width 0.2) (layer "F.Cu") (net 7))
 (segment (start 90.54 78.92) (end 90.54 36.04) (width 0.2) (layer "F.Cu") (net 7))
 (segment (start 118 124) (end 119 125) (width 0.2) (layer "F.Cu") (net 7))
 (segment (start 128.54 78.92) (end 128.54 73.54) (width 0.2) (layer "F.Cu") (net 7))
 (segment (start 91 22) (end 129 22) (width 0.2) (layer "F.Cu") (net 7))
 (segment (start 164.54 78.92) (end 164.54 73.54) (width 0.2) (layer "F.Cu") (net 7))
 (segment (start 152.08 129.92) (end 151 131) (width 0.2) (layer "F.Cu") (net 7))
 (segment (start 128.54 72) (end 128.54 73.54) (width 0.2) (layer "F.Cu") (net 7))
 (segment (start 202.54 72.54) (end 202 72) (width 0.2) (layer "F.Cu") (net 7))
 (segment (start 143 22) (end 130 22) (width 0.2) (layer "F.Cu") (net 7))
 (segment (start 119 151.78) (end 112.78 158) (width 0.2) (layer "F.Cu") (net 7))
 (segment (start 119 125) (end 119 151.78) (width 0.2) (layer "F.Cu") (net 7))
 (segment (start 222 31) (end 222 22) (width 0.2) (layer "F.Cu") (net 7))
 (segment (start 222 22) (end 220 20) (width 0.2) (layer "F.Cu") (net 7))
 (segment (start 64 152.78) (end 64 157.86) (width 0.2) (layer "F.Cu") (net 7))
 (segment (start 151 131) (end 151 154) (width 0.2) (layer "F.Cu") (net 7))
 (segment (start 151 50) (end 151 72) (width 0.2) (layer "F.Cu") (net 7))
 (segment (start 110 124) (end 118 124) (width 0.2) (layer "F.Cu") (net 7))
 (segment (start 129 22) (end 130 22) (width 0.2) (layer "F.Cu") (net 7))
 (segment (start 220 20) (end 200 20) (width 0.2) (layer "F.Cu") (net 7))
 (segment (start 200 30.5) (end 200 20) (width 0.2) (layer "F.Cu") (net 7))
 (segment (start 183.54 129.92) (end 152.08 129.92) (width 0.2) (layer "F.Cu") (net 7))
 (segment (start 93.92 140.08) (end 64 140.08) (width 0.2) (layer "F.Cu") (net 9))
 (segment (start 94 127) (end 94 140) (width 0.2) (layer "F.Cu") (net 9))
 (segment (start 115 122) (end 99 122) (width 0.2) (layer "F.Cu") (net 9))
 (segment (start 120.563655 81.46) (end 115 87.023655) (width 0.2) (layer "F.Cu") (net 9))
 (segment (start 122.19 81.46) (end 120.563655 81.46) (width 0.2) (layer "F.Cu") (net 9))
 (segment (start 99 122) (end 94 127) (width 0.2) (layer "F.Cu") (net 9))
 (segment (start 94 140) (end 93.92 140.08) (width 0.2) (layer "F.Cu") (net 9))
 (segment (start 115 87.023655) (end 115 122) (width 0.2) (layer "F.Cu") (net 9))
 (segment (start 149 20) (end 68 20) (width 0.2) (layer "F.Cu") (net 14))
 (segment (start 149.81 20.81) (end 149 20) (width 0.2) (layer "F.Cu") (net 14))
 (segment (start 64 24) (end 64 135) (width 0.2) (layer "F.Cu") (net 14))
 (segment (start 149.81 30.46) (end 149.81 20.81) (width 0.2) (layer "F.Cu") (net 14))
 (segment (start 68 20) (end 64 24) (width 0.2) (layer "F.Cu") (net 14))
 (segment (start 96 142) (end 95.38 142.62) (width 0.2) (layer "F.Cu") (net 13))
 (segment (start 96 134) (end 96 142) (width 0.2) (layer "F.Cu") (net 13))
 (segment (start 95.38 142.62) (end 64 142.62) (width 0.2) (layer "F.Cu") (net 13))
 (segment (start 103.19 132.46) (end 97.54 132.46) (width 0.2) (layer "F.Cu") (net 13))
 (segment (start 97.54 132.46) (end 96 134) (width 0.2) (layer "F.Cu") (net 13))
 (segment (start 67 35) (end 67 43) (width 0.2) (layer "B.Cu") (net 10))
 (segment (start 71 31) (end 67 35) (width 0.2) (layer "B.Cu") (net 10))
 (segment (start 73 44) (end 73 136.16) (width 0.2) (layer "B.Cu") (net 10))
 (segment (start 67 43) (end 72 43) (width 0.2) (layer "B.Cu") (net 10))
 (segment (start 73 136.16) (end 64 145.16) (width 0.2) (layer "B.Cu") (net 10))
 (segment (start 72 43) (end 73 44) (width 0.2) (layer "B.Cu") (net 10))
 (segment (start 71 130.54) (end 64 137.54) (width 0.2) (layer "F.Cu") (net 15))
 (segment (start 84.19 81.46) (end 72.54 81.46) (width 0.2) (layer "F.Cu") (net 15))
 (segment (start 72.54 81.46) (end 71 83) (width 0.2) (layer "F.Cu") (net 15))
 (segment (start 71 83) (end 71 130.54) (width 0.2) (layer "F.Cu") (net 15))
 (segment (start 75 43) (end 75 136.7) (width 0.2) (layer "B.Cu") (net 11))
 (segment (start 68 39) (end 68 42) (width 0.2) (layer "B.Cu") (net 11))
 (segment (start 68 42) (end 74 42) (width 0.2) (layer "B.Cu") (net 11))
 (segment (start 71 36) (end 68 39) (width 0.2) (layer "B.Cu") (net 11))
 (segment (start 74 42) (end 75 43) (width 0.2) (layer "B.Cu") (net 11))
 (segment (start 75 136.7) (end 64 147.7) (width 0.2) (layer "B.Cu") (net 11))
 (segment (start 201.46 132.46) (end 205 136) (width 0.2) (layer "B.Cu") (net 1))
 (segment (start 177.19 132.46) (end 201.46 132.46) (width 0.2) (layer "B.Cu") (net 1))
 (segment (start 205 136) (end 225 136) (width 0.2) (layer "B.Cu") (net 1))
 (segment (start 179 33) (end 176 36) (width 0.2) (layer "B.Cu") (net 5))
 (segment (start 200 33) (end 179 33) (width 0.2) (layer "B.Cu") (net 5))
 (segment (start 155 153) (end 218.16 153) (width 0.2) (layer "B.Cu") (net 5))
 (segment (start 176 36) (end 176 93) (width 0.2) (layer "B.Cu") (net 5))
 (segment (start 218.16 153) (end 225 146.16) (width 0.2) (layer "B.Cu") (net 5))
 (segment (start 156 97) (end 153 100) (width 0.2) (layer "B.Cu") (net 5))
 (segment (start 176 93) (end 172 97) (width 0.2) (layer "B.Cu") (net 5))
 (segment (start 203 36) (end 200 33) (width 0.2) (layer "B.Cu") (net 5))
 (segment (start 153 100) (end 153 151) (width 0.2) (layer "B.Cu") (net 5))
 (segment (start 172 97) (end 156 97) (width 0.2) (layer "B.Cu") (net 5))
 (segment (start 153 151) (end 155 153) (width 0.2) (layer "B.Cu") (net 5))
 (segment (start 154 102) (end 154 148) (width 0.2) (layer "B.Cu") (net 4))
 (segment (start 178 38) (end 178 93) (width 0.2) (layer "B.Cu") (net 4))
 (segment (start 181 35) (end 178 38) (width 0.2) (layer "B.Cu") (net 4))
 (segment (start 217.62 151) (end 225 143.62) (width 0.2) (layer "B.Cu") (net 4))
 (segment (start 154 148) (end 157 151) (width 0.2) (layer "B.Cu") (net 4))
 (segment (start 199 43) (end 199 37) (width 0.2) (layer "B.Cu") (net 4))
 (segment (start 157 99) (end 154 102) (width 0.2) (layer "B.Cu") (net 4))
 (segment (start 199 37) (end 197 35) (width 0.2) (layer "B.Cu") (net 4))
 (segment (start 172 99) (end 157 99) (width 0.2) (layer "B.Cu") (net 4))
 (segment (start 178 93) (end 172 99) (width 0.2) (layer "B.Cu") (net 4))
 (segment (start 221 45) (end 201 45) (width 0.2) (layer "B.Cu") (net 4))
 (segment (start 201 45) (end 199 43) (width 0.2) (layer "B.Cu") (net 4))
 (segment (start 197 35) (end 181 35) (width 0.2) (layer "B.Cu") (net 4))
 (segment (start 217.5 36) (end 221 39.5) (width 0.2) (layer "B.Cu") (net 4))
 (segment (start 221 39.5) (end 221 45) (width 0.2) (layer "B.Cu") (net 4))
 (segment (start 157 151) (end 217.62 151) (width 0.2) (layer "B.Cu") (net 4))
 (segment (start 200.54 138.54) (end 195 133) (width 0.2) (layer "F.Cu") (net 2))
 (segment (start 195 133) (end 195 114) (width 0.2) (layer "F.Cu") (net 2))
 (segment (start 189 108) (end 189 83) (width 0.2) (layer "F.Cu") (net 2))
 (segment (start 195 114) (end 189 108) (width 0.2) (layer "F.Cu") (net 2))
 (segment (start 190.54 81.46) (end 196.19 81.46) (width 0.2) (layer "F.Cu") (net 2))
 (segment (start 189 83) (end 190.54 81.46) (width 0.2) (layer "F.Cu") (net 2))
 (segment (start 225 138.54) (end 200.54 138.54) (width 0.2) (layer "F.Cu") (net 2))
 (segment (start 174 93) (end 174 35) (width 0.2) (layer "B.Cu") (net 6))
 (segment (start 152 99) (end 155 96) (width 0.2) (layer "B.Cu") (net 6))
 (segment (start 178 31) (end 203 31) (width 0.2) (layer "B.Cu") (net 6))
 (segment (start 219.7 154) (end 154 154) (width 0.2) (layer "B.Cu") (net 6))
 (segment (start 225 148.7) (end 219.7 154) (width 0.2) (layer "B.Cu") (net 6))
 (segment (start 171 96) (end 174 93) (width 0.2) (layer "B.Cu") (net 6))
 (segment (start 154 154) (end 152 152) (width 0.2) (layer "B.Cu") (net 6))
 (segment (start 152 152) (end 152 99) (width 0.2) (layer "B.Cu") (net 6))
 (segment (start 155 96) (end 171 96) (width 0.2) (layer "B.Cu") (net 6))
 (segment (start 174 35) (end 178 31) (width 0.2) (layer "B.Cu") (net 6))
 (segment (start 165 108) (end 185 108) (width 0.2) (layer "F.Cu") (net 3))
 (segment (start 193 136) (end 198.08 141.08) (width 0.2) (layer "F.Cu") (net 3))
 (segment (start 198.08 141.08) (end 225 141.08) (width 0.2) (layer "F.Cu") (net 3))
 (segment (start 185 108) (end 193 116) (width 0.2) (layer "F.Cu") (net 3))
 (segment (start 193 116) (end 193 136) (width 0.2) (layer "F.Cu") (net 3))
 (segment (start 158.19 81.46) (end 158.19 101.19) (width 0.2) (layer "F.Cu") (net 3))
 (segment (start 158.19 101.19) (end 165 108) (width 0.2) (layer "F.Cu") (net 3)))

